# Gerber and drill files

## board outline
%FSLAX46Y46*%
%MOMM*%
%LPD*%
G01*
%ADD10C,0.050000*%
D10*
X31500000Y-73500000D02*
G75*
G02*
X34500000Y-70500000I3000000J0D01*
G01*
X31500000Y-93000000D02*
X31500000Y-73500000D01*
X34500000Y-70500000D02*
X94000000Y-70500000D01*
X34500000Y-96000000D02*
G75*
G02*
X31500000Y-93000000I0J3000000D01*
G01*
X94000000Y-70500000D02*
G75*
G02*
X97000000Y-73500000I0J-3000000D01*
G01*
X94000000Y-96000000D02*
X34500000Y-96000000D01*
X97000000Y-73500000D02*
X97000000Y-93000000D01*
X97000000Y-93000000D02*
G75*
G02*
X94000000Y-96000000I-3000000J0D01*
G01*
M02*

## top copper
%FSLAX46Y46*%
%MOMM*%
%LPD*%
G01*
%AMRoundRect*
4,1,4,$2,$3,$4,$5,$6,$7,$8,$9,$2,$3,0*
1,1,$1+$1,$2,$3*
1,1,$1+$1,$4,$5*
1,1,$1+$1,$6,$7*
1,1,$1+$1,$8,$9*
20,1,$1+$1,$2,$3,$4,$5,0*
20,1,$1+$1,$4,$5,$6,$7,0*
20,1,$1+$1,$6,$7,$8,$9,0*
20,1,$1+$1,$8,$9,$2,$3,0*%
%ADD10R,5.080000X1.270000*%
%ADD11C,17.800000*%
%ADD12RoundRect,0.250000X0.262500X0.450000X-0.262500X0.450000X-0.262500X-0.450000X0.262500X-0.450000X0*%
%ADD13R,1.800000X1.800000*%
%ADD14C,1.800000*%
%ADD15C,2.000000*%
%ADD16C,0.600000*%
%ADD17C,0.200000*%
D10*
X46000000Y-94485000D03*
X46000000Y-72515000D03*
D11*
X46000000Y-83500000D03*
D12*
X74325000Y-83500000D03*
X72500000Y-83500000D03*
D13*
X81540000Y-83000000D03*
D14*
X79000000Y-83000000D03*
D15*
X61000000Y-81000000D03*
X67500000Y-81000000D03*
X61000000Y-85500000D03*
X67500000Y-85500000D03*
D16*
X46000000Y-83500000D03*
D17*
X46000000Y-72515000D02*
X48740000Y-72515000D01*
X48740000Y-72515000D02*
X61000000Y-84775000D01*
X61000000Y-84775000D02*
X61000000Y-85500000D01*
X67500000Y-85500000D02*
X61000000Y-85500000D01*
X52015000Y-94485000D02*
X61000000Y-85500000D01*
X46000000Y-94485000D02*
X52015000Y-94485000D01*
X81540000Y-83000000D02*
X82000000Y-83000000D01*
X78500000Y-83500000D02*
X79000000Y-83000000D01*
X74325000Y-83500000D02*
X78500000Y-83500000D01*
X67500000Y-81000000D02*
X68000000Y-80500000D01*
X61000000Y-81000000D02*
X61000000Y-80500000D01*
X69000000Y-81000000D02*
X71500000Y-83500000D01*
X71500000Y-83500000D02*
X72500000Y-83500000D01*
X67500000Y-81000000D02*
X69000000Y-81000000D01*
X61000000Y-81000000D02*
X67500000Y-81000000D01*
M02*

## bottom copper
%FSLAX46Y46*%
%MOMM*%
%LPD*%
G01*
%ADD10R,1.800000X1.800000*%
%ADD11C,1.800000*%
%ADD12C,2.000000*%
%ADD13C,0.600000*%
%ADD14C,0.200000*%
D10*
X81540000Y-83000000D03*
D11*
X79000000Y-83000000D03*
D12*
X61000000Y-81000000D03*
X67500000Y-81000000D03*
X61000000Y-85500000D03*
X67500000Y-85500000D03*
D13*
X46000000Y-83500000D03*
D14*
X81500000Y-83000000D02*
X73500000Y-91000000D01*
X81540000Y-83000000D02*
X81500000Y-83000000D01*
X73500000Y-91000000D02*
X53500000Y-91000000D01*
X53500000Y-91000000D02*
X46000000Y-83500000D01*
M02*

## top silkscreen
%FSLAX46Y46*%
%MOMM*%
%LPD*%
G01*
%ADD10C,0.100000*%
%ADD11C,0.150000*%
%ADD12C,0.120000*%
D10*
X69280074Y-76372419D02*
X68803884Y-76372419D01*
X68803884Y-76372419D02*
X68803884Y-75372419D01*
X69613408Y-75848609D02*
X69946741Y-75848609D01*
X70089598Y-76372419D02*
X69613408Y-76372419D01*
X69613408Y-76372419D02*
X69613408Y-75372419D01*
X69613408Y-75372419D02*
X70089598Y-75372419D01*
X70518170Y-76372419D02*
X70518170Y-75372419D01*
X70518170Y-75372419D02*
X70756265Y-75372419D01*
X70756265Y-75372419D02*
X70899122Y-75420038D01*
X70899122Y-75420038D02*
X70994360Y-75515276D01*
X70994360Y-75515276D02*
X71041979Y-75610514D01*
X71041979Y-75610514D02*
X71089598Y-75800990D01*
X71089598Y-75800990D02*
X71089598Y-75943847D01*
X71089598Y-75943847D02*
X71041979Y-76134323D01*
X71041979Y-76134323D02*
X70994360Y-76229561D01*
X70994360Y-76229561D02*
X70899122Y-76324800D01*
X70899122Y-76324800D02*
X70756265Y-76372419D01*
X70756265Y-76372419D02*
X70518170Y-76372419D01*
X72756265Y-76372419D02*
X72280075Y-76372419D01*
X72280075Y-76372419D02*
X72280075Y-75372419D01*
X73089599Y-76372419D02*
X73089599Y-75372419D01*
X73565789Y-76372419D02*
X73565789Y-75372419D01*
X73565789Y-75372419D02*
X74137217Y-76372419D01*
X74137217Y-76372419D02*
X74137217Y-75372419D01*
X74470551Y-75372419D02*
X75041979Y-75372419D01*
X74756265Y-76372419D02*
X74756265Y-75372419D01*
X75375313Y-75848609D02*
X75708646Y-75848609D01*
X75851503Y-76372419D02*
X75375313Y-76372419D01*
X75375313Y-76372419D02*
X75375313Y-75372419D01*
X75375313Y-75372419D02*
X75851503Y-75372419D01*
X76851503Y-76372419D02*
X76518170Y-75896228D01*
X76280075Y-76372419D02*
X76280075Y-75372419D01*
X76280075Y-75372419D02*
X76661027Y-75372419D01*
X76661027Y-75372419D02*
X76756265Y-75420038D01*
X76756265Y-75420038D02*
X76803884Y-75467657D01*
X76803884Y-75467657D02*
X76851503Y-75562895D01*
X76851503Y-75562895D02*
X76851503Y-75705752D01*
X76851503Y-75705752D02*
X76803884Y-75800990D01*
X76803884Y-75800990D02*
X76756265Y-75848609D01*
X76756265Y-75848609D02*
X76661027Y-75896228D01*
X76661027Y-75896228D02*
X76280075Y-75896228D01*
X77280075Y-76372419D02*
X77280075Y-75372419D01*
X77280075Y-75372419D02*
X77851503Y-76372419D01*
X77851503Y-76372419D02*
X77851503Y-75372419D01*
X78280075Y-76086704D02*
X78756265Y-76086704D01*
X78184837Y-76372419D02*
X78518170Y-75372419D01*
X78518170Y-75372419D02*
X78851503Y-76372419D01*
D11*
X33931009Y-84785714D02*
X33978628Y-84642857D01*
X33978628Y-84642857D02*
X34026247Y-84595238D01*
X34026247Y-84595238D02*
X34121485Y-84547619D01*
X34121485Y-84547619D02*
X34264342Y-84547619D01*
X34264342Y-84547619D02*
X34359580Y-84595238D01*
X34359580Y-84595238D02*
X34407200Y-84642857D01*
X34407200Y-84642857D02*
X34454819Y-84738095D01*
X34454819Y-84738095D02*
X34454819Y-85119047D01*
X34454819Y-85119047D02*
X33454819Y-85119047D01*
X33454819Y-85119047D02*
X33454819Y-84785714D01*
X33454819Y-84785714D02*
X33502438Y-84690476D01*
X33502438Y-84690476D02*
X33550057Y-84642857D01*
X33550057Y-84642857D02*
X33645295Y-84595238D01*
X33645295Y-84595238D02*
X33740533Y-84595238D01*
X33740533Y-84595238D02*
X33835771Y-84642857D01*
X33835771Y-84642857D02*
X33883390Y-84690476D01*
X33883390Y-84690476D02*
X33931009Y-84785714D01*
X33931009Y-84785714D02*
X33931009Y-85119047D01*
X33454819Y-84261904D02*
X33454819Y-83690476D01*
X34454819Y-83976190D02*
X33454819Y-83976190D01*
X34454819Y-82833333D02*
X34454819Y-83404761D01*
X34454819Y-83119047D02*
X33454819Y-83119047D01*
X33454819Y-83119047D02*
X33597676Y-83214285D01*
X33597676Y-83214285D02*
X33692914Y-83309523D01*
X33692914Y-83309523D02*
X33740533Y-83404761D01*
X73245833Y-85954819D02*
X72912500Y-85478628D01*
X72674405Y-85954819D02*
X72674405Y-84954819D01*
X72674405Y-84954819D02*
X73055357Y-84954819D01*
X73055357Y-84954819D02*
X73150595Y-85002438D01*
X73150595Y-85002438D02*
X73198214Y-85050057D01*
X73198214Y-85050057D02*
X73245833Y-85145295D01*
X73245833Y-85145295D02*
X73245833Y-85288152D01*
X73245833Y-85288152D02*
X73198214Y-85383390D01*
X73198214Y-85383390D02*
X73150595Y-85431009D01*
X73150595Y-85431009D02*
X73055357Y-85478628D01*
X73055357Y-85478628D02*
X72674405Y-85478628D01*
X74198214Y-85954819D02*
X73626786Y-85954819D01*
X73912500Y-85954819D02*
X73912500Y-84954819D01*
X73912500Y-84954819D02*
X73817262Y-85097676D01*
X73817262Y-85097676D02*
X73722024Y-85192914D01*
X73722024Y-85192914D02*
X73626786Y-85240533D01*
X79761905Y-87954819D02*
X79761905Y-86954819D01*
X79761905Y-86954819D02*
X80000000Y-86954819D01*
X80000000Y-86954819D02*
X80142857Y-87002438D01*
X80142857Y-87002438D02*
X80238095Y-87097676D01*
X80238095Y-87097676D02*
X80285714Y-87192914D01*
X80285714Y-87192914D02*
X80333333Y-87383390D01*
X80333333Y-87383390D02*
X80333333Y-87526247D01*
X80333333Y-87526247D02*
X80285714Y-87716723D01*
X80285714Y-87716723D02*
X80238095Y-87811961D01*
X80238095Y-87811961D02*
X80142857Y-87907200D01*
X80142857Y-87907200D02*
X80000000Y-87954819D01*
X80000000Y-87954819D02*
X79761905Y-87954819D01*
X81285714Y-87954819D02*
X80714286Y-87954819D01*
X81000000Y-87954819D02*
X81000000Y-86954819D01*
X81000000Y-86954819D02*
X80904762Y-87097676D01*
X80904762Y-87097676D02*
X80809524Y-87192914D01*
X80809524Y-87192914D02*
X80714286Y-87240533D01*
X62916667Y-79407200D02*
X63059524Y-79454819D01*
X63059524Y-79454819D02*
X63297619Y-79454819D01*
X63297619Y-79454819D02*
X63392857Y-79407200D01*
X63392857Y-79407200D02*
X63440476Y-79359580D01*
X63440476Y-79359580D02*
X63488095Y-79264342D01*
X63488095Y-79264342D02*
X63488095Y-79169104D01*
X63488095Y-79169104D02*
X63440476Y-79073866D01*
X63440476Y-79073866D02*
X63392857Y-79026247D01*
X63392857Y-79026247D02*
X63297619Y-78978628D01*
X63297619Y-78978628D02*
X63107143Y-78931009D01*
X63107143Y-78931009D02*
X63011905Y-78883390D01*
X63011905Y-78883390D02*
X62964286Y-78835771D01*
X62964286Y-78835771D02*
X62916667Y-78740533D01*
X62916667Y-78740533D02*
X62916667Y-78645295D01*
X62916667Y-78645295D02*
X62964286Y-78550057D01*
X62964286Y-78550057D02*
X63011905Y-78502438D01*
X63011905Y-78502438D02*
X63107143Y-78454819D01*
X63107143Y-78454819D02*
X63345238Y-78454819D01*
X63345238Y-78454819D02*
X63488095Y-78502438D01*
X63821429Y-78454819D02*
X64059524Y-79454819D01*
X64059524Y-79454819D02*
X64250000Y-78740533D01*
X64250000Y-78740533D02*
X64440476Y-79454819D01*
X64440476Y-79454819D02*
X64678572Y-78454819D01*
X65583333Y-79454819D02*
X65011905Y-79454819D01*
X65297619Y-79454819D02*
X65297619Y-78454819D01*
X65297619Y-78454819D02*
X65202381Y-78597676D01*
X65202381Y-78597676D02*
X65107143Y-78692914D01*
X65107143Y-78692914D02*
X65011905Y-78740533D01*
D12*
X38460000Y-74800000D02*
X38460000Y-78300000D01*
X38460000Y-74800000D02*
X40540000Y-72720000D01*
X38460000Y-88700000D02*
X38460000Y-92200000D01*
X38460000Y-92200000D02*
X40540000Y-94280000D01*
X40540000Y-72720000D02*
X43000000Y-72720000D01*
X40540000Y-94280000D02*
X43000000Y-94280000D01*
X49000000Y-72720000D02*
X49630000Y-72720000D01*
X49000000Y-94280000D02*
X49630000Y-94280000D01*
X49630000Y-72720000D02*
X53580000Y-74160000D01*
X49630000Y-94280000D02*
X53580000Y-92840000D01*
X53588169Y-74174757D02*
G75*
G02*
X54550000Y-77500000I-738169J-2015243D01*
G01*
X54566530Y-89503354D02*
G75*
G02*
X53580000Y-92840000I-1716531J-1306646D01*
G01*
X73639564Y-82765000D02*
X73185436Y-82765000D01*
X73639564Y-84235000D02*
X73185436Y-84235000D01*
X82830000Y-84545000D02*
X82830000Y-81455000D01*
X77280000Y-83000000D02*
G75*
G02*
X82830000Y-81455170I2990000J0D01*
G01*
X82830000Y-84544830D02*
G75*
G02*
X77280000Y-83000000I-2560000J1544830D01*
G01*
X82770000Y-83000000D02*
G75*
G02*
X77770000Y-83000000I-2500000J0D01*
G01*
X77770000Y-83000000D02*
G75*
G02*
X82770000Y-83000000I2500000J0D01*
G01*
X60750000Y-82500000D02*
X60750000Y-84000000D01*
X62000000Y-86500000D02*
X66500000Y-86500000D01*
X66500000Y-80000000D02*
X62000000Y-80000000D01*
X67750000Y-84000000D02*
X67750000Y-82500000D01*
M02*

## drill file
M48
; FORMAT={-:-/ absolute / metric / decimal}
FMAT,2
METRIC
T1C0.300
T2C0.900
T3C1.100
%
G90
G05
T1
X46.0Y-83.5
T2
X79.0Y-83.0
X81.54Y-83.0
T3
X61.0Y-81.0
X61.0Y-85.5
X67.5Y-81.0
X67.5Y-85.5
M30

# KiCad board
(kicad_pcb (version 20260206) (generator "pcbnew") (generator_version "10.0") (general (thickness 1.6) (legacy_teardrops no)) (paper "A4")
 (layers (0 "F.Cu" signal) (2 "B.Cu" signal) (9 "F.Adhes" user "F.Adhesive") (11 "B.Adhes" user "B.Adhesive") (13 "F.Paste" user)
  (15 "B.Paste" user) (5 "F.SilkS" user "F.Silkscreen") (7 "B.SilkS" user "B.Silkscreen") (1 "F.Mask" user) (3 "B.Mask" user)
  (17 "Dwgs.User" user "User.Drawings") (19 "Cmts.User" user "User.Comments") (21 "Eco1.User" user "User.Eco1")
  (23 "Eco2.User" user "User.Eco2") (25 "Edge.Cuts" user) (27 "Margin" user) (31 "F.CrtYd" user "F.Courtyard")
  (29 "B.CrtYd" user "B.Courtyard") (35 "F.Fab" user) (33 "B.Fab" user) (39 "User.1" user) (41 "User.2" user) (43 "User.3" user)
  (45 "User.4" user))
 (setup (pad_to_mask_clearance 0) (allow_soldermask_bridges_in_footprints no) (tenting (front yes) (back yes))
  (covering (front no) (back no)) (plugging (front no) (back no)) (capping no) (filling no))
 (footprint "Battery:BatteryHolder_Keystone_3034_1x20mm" (layer "F.Cu") (at 46 83.5 90)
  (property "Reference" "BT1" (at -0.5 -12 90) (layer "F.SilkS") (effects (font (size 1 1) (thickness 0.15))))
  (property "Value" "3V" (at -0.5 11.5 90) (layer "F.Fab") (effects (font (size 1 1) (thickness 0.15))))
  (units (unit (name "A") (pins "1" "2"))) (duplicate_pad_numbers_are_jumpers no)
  (fp_line (start 8.7 -7.54) (end 5.2 -7.54) (stroke (width 0.12) (type solid)) (layer "F.SilkS"))
  (fp_line (start 8.7 -7.54) (end 10.78 -5.46) (stroke (width 0.12) (type solid)) (layer "F.SilkS"))
  (fp_line (start -5.2 -7.54) (end -8.7 -7.54) (stroke (width 0.12) (type solid)) (layer "F.SilkS"))
  (fp_line (start -8.7 -7.54) (end -10.78 -5.46) (stroke (width 0.12) (type solid)) (layer "F.SilkS"))
  (fp_line (start 10.78 -5.46) (end 10.78 -3) (stroke (width 0.12) (type solid)) (layer "F.SilkS"))
  (fp_line (start -10.78 -5.46) (end -10.78 -3) (stroke (width 0.12) (type solid)) (layer "F.SilkS"))
  (fp_line (start 10.78 3) (end 10.78 3.63) (stroke (width 0.12) (type solid)) (layer "F.SilkS"))
  (fp_line (start -10.78 3) (end -10.78 3.63) (stroke (width 0.12) (type solid)) (layer "F.SilkS"))
  (fp_line (start 10.78 3.63) (end 9.34 7.58) (stroke (width 0.12) (type solid)) (layer "F.SilkS"))
  (fp_line (start -10.78 3.63) (end -9.34 7.58) (stroke (width 0.12) (type solid)) (layer "F.SilkS"))
  (fp_arc (start 9.325243 7.588169) (mid 7.90634 8.911668) (end 6 8.55) (stroke (width 0.12) (type solid)) (layer "F.SilkS"))
  (fp_arc (start -6.003354 8.56653) (mid -7.921654 8.918738) (end -9.34 7.58) (stroke (width 0.12) (type solid)) (layer "F.SilkS"))
  (pad "1" smd rect (at -10.985 0 90) (size 1.27 5.08) (layers "F.Cu" "F.Mask" "F.Paste") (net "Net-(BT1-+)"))
  (pad "1" smd rect (at 10.985 0 90) (size 1.27 5.08) (layers "F.Cu" "F.Mask" "F.Paste") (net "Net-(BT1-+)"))
  (pad "2" smd circle (at 0 0 90) (size 17.8 17.8) (layers "F.Cu" "F.Mask") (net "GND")))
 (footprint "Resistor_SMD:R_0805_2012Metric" (layer "F.Cu") (at 73.4125 83.5 180)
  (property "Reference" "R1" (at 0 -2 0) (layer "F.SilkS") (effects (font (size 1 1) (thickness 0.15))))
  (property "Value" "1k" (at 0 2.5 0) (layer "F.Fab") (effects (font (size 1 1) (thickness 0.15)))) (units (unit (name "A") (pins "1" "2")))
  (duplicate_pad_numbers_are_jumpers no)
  (fp_line (start -0.227064 0.735) (end 0.227064 0.735) (stroke (width 0.12) (type solid)) (layer "F.SilkS"))
  (fp_line (start -0.227064 -0.735) (end 0.227064 -0.735) (stroke (width 0.12) (type solid)) (layer "F.SilkS"))
  (pad "1" smd roundrect (at -0.9125 0 180) (size 1.025 1.4) (layers "F.Cu" "F.Mask" "F.Paste") (roundrect_rratio 0.243902)
   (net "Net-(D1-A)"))
  (pad "2" smd roundrect (at 0.9125 0 180) (size 1.025 1.4) (layers "F.Cu" "F.Mask" "F.Paste") (roundrect_rratio 0.243902)
   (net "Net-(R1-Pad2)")))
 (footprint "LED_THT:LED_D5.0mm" (layer "F.Cu") (at 81.54 83 180)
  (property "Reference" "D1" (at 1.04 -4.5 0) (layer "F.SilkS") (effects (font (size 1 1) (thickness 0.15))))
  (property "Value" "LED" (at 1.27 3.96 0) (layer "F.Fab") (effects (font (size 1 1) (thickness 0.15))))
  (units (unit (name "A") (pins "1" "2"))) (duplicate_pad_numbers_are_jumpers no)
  (fp_line (start -1.29 -1.545) (end -1.29 1.545) (stroke (width 0.12) (type solid)) (layer "F.SilkS"))
  (fp_arc (start 4.26 0) (mid 2.071779 2.880495) (end -1.29 1.54483) (stroke (width 0.12) (type solid)) (layer "F.SilkS"))
  (fp_arc (start -1.29 -1.54483) (mid 2.071779 -2.880495) (end 4.26 0) (stroke (width 0.12) (type solid)) (layer "F.SilkS"))
  (fp_circle (center 1.27 0) (end 3.77 0) (stroke (width 0.12) (type solid)) (fill no) (layer "F.SilkS"))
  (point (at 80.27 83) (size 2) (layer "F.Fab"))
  (pad "1" thru_hole rect (at 0 0 180) (size 1.8 1.8) (drill 0.9) (layers "*.Cu" "*.Mask") (remove_unused_layers no) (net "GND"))
  (pad "2" thru_hole circle (at 2.54 0 180) (size 1.8 1.8) (drill 0.9) (layers "*.Cu" "*.Mask") (remove_unused_layers no) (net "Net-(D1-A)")))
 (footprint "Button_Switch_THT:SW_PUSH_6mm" (layer "F.Cu") (at 61 81)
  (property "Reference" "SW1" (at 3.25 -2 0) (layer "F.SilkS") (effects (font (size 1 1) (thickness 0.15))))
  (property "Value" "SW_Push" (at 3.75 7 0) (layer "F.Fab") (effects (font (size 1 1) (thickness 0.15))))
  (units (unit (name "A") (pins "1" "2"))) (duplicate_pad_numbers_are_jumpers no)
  (fp_line (start -0.25 1.5) (end -0.25 3) (stroke (width 0.12) (type solid)) (layer "F.SilkS"))
  (fp_line (start 1 5.5) (end 5.5 5.5) (stroke (width 0.12) (type solid)) (layer "F.SilkS"))
  (fp_line (start 5.5 -1) (end 1 -1) (stroke (width 0.12) (type solid)) (layer "F.SilkS"))
  (fp_line (start 6.75 3) (end 6.75 1.5) (stroke (width 0.12) (type solid)) (layer "F.SilkS"))
  (pad "1" thru_hole circle (at 0 0 90) (size 2 2) (drill 1.1) (layers "*.Cu" "*.Mask") (remove_unused_layers no) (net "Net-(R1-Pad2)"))
  (pad "1" thru_hole circle (at 6.5 0 90) (size 2 2) (drill 1.1) (layers "*.Cu" "*.Mask") (remove_unused_layers no) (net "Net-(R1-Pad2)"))
  (pad "2" thru_hole circle (at 0 4.5 90) (size 2 2) (drill 1.1) (layers "*.Cu" "*.Mask") (remove_unused_layers no) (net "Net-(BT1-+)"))
  (pad "2" thru_hole circle (at 6.5 4.5 90) (size 2 2) (drill 1.1) (layers "*.Cu" "*.Mask") (remove_unused_layers no) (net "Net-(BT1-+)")))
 (gr_arc (start 31.5 73.5) (mid 32.37868 71.37868) (end 34.5 70.5) (stroke (width 0.05) (type default)) (layer "Edge.Cuts"))
 (gr_line (start 31.5 93) (end 31.5 73.5) (stroke (width 0.05) (type default)) (layer "Edge.Cuts"))
 (gr_line (start 34.5 70.5) (end 94 70.5) (stroke (width 0.05) (type default)) (layer "Edge.Cuts"))
 (gr_arc (start 34.5 96) (mid 32.37868 95.12132) (end 31.5 93) (stroke (width 0.05) (type default)) (layer "Edge.Cuts"))
 (gr_arc (start 94 70.5) (mid 96.12132 71.37868) (end 97 73.5) (stroke (width 0.05) (type default)) (layer "Edge.Cuts"))
 (gr_line (start 94 96) (end 34.5 96) (stroke (width 0.05) (type default)) (layer "Edge.Cuts"))
 (gr_line (start 97 73.5) (end 97 93) (stroke (width 0.05) (type default)) (layer "Edge.Cuts"))
 (gr_arc (start 97 93) (mid 96.12132 95.12132) (end 94 96) (stroke (width 0.05) (type default)) (layer "Edge.Cuts"))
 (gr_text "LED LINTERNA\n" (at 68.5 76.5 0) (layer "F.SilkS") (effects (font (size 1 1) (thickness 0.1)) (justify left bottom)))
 (segment (start 46 72.515) (end 48.74 72.515) (width 0.2) (layer "F.Cu") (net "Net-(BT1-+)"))
 (segment (start 48.74 72.515) (end 61 84.775) (width 0.2) (layer "F.Cu") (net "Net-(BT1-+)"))
 (segment (start 61 84.775) (end 61 85.5) (width 0.2) (layer "F.Cu") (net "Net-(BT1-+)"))
 (segment (start 67.5 85.5) (end 61 85.5) (width 0.2) (layer "F.Cu") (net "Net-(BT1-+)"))
 (segment (start 52.015 94.485) (end 61 85.5) (width 0.2) (layer "F.Cu") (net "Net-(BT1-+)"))
 (segment (start 46 94.485) (end 52.015 94.485) (width 0.2) (layer "F.Cu") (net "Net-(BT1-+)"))
 (segment (start 81.54 83) (end 82 83) (width 0.2) (layer "F.Cu") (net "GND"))
 (via (at 46 83.5) (size 0.6) (drill 0.3) (layers "F.Cu" "B.Cu") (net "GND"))
 (segment (start 81.5 83) (end 73.5 91) (width 0.2) (layer "B.Cu") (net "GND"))
 (segment (start 81.54 83) (end 81.5 83) (width 0.2) (layer "B.Cu") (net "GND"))
 (segment (start 73.5 91) (end 53.5 91) (width 0.2) (layer "B.Cu") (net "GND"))
 (segment (start 53.5 91) (end 46 83.5) (width 0.2) (layer "B.Cu") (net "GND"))
 (segment (start 78.5 83.5) (end 79 83) (width 0.2) (layer "F.Cu") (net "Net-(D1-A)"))
 (segment (start 74.325 83.5) (end 78.5 83.5) (width 0.2) (layer "F.Cu") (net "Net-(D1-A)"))
 (segment (start 67.5 81) (end 68 80.5) (width 0.2) (layer "F.Cu") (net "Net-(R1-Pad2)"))
 (segment (start 61 81) (end 61 80.5) (width 0.2) (layer "F.Cu") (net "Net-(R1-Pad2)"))
 (segment (start 69 81) (end 71.5 83.5) (width 0.2) (layer "F.Cu") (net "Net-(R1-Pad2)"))
 (segment (start 71.5 83.5) (end 72.5 83.5) (width 0.2) (layer "F.Cu") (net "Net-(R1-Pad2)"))
 (segment (start 67.5 81) (end 69 81) (width 0.2) (layer "F.Cu") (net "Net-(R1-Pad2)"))
 (segment (start 61 81) (end 67.5 81) (width 0.2) (layer "F.Cu") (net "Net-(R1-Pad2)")))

